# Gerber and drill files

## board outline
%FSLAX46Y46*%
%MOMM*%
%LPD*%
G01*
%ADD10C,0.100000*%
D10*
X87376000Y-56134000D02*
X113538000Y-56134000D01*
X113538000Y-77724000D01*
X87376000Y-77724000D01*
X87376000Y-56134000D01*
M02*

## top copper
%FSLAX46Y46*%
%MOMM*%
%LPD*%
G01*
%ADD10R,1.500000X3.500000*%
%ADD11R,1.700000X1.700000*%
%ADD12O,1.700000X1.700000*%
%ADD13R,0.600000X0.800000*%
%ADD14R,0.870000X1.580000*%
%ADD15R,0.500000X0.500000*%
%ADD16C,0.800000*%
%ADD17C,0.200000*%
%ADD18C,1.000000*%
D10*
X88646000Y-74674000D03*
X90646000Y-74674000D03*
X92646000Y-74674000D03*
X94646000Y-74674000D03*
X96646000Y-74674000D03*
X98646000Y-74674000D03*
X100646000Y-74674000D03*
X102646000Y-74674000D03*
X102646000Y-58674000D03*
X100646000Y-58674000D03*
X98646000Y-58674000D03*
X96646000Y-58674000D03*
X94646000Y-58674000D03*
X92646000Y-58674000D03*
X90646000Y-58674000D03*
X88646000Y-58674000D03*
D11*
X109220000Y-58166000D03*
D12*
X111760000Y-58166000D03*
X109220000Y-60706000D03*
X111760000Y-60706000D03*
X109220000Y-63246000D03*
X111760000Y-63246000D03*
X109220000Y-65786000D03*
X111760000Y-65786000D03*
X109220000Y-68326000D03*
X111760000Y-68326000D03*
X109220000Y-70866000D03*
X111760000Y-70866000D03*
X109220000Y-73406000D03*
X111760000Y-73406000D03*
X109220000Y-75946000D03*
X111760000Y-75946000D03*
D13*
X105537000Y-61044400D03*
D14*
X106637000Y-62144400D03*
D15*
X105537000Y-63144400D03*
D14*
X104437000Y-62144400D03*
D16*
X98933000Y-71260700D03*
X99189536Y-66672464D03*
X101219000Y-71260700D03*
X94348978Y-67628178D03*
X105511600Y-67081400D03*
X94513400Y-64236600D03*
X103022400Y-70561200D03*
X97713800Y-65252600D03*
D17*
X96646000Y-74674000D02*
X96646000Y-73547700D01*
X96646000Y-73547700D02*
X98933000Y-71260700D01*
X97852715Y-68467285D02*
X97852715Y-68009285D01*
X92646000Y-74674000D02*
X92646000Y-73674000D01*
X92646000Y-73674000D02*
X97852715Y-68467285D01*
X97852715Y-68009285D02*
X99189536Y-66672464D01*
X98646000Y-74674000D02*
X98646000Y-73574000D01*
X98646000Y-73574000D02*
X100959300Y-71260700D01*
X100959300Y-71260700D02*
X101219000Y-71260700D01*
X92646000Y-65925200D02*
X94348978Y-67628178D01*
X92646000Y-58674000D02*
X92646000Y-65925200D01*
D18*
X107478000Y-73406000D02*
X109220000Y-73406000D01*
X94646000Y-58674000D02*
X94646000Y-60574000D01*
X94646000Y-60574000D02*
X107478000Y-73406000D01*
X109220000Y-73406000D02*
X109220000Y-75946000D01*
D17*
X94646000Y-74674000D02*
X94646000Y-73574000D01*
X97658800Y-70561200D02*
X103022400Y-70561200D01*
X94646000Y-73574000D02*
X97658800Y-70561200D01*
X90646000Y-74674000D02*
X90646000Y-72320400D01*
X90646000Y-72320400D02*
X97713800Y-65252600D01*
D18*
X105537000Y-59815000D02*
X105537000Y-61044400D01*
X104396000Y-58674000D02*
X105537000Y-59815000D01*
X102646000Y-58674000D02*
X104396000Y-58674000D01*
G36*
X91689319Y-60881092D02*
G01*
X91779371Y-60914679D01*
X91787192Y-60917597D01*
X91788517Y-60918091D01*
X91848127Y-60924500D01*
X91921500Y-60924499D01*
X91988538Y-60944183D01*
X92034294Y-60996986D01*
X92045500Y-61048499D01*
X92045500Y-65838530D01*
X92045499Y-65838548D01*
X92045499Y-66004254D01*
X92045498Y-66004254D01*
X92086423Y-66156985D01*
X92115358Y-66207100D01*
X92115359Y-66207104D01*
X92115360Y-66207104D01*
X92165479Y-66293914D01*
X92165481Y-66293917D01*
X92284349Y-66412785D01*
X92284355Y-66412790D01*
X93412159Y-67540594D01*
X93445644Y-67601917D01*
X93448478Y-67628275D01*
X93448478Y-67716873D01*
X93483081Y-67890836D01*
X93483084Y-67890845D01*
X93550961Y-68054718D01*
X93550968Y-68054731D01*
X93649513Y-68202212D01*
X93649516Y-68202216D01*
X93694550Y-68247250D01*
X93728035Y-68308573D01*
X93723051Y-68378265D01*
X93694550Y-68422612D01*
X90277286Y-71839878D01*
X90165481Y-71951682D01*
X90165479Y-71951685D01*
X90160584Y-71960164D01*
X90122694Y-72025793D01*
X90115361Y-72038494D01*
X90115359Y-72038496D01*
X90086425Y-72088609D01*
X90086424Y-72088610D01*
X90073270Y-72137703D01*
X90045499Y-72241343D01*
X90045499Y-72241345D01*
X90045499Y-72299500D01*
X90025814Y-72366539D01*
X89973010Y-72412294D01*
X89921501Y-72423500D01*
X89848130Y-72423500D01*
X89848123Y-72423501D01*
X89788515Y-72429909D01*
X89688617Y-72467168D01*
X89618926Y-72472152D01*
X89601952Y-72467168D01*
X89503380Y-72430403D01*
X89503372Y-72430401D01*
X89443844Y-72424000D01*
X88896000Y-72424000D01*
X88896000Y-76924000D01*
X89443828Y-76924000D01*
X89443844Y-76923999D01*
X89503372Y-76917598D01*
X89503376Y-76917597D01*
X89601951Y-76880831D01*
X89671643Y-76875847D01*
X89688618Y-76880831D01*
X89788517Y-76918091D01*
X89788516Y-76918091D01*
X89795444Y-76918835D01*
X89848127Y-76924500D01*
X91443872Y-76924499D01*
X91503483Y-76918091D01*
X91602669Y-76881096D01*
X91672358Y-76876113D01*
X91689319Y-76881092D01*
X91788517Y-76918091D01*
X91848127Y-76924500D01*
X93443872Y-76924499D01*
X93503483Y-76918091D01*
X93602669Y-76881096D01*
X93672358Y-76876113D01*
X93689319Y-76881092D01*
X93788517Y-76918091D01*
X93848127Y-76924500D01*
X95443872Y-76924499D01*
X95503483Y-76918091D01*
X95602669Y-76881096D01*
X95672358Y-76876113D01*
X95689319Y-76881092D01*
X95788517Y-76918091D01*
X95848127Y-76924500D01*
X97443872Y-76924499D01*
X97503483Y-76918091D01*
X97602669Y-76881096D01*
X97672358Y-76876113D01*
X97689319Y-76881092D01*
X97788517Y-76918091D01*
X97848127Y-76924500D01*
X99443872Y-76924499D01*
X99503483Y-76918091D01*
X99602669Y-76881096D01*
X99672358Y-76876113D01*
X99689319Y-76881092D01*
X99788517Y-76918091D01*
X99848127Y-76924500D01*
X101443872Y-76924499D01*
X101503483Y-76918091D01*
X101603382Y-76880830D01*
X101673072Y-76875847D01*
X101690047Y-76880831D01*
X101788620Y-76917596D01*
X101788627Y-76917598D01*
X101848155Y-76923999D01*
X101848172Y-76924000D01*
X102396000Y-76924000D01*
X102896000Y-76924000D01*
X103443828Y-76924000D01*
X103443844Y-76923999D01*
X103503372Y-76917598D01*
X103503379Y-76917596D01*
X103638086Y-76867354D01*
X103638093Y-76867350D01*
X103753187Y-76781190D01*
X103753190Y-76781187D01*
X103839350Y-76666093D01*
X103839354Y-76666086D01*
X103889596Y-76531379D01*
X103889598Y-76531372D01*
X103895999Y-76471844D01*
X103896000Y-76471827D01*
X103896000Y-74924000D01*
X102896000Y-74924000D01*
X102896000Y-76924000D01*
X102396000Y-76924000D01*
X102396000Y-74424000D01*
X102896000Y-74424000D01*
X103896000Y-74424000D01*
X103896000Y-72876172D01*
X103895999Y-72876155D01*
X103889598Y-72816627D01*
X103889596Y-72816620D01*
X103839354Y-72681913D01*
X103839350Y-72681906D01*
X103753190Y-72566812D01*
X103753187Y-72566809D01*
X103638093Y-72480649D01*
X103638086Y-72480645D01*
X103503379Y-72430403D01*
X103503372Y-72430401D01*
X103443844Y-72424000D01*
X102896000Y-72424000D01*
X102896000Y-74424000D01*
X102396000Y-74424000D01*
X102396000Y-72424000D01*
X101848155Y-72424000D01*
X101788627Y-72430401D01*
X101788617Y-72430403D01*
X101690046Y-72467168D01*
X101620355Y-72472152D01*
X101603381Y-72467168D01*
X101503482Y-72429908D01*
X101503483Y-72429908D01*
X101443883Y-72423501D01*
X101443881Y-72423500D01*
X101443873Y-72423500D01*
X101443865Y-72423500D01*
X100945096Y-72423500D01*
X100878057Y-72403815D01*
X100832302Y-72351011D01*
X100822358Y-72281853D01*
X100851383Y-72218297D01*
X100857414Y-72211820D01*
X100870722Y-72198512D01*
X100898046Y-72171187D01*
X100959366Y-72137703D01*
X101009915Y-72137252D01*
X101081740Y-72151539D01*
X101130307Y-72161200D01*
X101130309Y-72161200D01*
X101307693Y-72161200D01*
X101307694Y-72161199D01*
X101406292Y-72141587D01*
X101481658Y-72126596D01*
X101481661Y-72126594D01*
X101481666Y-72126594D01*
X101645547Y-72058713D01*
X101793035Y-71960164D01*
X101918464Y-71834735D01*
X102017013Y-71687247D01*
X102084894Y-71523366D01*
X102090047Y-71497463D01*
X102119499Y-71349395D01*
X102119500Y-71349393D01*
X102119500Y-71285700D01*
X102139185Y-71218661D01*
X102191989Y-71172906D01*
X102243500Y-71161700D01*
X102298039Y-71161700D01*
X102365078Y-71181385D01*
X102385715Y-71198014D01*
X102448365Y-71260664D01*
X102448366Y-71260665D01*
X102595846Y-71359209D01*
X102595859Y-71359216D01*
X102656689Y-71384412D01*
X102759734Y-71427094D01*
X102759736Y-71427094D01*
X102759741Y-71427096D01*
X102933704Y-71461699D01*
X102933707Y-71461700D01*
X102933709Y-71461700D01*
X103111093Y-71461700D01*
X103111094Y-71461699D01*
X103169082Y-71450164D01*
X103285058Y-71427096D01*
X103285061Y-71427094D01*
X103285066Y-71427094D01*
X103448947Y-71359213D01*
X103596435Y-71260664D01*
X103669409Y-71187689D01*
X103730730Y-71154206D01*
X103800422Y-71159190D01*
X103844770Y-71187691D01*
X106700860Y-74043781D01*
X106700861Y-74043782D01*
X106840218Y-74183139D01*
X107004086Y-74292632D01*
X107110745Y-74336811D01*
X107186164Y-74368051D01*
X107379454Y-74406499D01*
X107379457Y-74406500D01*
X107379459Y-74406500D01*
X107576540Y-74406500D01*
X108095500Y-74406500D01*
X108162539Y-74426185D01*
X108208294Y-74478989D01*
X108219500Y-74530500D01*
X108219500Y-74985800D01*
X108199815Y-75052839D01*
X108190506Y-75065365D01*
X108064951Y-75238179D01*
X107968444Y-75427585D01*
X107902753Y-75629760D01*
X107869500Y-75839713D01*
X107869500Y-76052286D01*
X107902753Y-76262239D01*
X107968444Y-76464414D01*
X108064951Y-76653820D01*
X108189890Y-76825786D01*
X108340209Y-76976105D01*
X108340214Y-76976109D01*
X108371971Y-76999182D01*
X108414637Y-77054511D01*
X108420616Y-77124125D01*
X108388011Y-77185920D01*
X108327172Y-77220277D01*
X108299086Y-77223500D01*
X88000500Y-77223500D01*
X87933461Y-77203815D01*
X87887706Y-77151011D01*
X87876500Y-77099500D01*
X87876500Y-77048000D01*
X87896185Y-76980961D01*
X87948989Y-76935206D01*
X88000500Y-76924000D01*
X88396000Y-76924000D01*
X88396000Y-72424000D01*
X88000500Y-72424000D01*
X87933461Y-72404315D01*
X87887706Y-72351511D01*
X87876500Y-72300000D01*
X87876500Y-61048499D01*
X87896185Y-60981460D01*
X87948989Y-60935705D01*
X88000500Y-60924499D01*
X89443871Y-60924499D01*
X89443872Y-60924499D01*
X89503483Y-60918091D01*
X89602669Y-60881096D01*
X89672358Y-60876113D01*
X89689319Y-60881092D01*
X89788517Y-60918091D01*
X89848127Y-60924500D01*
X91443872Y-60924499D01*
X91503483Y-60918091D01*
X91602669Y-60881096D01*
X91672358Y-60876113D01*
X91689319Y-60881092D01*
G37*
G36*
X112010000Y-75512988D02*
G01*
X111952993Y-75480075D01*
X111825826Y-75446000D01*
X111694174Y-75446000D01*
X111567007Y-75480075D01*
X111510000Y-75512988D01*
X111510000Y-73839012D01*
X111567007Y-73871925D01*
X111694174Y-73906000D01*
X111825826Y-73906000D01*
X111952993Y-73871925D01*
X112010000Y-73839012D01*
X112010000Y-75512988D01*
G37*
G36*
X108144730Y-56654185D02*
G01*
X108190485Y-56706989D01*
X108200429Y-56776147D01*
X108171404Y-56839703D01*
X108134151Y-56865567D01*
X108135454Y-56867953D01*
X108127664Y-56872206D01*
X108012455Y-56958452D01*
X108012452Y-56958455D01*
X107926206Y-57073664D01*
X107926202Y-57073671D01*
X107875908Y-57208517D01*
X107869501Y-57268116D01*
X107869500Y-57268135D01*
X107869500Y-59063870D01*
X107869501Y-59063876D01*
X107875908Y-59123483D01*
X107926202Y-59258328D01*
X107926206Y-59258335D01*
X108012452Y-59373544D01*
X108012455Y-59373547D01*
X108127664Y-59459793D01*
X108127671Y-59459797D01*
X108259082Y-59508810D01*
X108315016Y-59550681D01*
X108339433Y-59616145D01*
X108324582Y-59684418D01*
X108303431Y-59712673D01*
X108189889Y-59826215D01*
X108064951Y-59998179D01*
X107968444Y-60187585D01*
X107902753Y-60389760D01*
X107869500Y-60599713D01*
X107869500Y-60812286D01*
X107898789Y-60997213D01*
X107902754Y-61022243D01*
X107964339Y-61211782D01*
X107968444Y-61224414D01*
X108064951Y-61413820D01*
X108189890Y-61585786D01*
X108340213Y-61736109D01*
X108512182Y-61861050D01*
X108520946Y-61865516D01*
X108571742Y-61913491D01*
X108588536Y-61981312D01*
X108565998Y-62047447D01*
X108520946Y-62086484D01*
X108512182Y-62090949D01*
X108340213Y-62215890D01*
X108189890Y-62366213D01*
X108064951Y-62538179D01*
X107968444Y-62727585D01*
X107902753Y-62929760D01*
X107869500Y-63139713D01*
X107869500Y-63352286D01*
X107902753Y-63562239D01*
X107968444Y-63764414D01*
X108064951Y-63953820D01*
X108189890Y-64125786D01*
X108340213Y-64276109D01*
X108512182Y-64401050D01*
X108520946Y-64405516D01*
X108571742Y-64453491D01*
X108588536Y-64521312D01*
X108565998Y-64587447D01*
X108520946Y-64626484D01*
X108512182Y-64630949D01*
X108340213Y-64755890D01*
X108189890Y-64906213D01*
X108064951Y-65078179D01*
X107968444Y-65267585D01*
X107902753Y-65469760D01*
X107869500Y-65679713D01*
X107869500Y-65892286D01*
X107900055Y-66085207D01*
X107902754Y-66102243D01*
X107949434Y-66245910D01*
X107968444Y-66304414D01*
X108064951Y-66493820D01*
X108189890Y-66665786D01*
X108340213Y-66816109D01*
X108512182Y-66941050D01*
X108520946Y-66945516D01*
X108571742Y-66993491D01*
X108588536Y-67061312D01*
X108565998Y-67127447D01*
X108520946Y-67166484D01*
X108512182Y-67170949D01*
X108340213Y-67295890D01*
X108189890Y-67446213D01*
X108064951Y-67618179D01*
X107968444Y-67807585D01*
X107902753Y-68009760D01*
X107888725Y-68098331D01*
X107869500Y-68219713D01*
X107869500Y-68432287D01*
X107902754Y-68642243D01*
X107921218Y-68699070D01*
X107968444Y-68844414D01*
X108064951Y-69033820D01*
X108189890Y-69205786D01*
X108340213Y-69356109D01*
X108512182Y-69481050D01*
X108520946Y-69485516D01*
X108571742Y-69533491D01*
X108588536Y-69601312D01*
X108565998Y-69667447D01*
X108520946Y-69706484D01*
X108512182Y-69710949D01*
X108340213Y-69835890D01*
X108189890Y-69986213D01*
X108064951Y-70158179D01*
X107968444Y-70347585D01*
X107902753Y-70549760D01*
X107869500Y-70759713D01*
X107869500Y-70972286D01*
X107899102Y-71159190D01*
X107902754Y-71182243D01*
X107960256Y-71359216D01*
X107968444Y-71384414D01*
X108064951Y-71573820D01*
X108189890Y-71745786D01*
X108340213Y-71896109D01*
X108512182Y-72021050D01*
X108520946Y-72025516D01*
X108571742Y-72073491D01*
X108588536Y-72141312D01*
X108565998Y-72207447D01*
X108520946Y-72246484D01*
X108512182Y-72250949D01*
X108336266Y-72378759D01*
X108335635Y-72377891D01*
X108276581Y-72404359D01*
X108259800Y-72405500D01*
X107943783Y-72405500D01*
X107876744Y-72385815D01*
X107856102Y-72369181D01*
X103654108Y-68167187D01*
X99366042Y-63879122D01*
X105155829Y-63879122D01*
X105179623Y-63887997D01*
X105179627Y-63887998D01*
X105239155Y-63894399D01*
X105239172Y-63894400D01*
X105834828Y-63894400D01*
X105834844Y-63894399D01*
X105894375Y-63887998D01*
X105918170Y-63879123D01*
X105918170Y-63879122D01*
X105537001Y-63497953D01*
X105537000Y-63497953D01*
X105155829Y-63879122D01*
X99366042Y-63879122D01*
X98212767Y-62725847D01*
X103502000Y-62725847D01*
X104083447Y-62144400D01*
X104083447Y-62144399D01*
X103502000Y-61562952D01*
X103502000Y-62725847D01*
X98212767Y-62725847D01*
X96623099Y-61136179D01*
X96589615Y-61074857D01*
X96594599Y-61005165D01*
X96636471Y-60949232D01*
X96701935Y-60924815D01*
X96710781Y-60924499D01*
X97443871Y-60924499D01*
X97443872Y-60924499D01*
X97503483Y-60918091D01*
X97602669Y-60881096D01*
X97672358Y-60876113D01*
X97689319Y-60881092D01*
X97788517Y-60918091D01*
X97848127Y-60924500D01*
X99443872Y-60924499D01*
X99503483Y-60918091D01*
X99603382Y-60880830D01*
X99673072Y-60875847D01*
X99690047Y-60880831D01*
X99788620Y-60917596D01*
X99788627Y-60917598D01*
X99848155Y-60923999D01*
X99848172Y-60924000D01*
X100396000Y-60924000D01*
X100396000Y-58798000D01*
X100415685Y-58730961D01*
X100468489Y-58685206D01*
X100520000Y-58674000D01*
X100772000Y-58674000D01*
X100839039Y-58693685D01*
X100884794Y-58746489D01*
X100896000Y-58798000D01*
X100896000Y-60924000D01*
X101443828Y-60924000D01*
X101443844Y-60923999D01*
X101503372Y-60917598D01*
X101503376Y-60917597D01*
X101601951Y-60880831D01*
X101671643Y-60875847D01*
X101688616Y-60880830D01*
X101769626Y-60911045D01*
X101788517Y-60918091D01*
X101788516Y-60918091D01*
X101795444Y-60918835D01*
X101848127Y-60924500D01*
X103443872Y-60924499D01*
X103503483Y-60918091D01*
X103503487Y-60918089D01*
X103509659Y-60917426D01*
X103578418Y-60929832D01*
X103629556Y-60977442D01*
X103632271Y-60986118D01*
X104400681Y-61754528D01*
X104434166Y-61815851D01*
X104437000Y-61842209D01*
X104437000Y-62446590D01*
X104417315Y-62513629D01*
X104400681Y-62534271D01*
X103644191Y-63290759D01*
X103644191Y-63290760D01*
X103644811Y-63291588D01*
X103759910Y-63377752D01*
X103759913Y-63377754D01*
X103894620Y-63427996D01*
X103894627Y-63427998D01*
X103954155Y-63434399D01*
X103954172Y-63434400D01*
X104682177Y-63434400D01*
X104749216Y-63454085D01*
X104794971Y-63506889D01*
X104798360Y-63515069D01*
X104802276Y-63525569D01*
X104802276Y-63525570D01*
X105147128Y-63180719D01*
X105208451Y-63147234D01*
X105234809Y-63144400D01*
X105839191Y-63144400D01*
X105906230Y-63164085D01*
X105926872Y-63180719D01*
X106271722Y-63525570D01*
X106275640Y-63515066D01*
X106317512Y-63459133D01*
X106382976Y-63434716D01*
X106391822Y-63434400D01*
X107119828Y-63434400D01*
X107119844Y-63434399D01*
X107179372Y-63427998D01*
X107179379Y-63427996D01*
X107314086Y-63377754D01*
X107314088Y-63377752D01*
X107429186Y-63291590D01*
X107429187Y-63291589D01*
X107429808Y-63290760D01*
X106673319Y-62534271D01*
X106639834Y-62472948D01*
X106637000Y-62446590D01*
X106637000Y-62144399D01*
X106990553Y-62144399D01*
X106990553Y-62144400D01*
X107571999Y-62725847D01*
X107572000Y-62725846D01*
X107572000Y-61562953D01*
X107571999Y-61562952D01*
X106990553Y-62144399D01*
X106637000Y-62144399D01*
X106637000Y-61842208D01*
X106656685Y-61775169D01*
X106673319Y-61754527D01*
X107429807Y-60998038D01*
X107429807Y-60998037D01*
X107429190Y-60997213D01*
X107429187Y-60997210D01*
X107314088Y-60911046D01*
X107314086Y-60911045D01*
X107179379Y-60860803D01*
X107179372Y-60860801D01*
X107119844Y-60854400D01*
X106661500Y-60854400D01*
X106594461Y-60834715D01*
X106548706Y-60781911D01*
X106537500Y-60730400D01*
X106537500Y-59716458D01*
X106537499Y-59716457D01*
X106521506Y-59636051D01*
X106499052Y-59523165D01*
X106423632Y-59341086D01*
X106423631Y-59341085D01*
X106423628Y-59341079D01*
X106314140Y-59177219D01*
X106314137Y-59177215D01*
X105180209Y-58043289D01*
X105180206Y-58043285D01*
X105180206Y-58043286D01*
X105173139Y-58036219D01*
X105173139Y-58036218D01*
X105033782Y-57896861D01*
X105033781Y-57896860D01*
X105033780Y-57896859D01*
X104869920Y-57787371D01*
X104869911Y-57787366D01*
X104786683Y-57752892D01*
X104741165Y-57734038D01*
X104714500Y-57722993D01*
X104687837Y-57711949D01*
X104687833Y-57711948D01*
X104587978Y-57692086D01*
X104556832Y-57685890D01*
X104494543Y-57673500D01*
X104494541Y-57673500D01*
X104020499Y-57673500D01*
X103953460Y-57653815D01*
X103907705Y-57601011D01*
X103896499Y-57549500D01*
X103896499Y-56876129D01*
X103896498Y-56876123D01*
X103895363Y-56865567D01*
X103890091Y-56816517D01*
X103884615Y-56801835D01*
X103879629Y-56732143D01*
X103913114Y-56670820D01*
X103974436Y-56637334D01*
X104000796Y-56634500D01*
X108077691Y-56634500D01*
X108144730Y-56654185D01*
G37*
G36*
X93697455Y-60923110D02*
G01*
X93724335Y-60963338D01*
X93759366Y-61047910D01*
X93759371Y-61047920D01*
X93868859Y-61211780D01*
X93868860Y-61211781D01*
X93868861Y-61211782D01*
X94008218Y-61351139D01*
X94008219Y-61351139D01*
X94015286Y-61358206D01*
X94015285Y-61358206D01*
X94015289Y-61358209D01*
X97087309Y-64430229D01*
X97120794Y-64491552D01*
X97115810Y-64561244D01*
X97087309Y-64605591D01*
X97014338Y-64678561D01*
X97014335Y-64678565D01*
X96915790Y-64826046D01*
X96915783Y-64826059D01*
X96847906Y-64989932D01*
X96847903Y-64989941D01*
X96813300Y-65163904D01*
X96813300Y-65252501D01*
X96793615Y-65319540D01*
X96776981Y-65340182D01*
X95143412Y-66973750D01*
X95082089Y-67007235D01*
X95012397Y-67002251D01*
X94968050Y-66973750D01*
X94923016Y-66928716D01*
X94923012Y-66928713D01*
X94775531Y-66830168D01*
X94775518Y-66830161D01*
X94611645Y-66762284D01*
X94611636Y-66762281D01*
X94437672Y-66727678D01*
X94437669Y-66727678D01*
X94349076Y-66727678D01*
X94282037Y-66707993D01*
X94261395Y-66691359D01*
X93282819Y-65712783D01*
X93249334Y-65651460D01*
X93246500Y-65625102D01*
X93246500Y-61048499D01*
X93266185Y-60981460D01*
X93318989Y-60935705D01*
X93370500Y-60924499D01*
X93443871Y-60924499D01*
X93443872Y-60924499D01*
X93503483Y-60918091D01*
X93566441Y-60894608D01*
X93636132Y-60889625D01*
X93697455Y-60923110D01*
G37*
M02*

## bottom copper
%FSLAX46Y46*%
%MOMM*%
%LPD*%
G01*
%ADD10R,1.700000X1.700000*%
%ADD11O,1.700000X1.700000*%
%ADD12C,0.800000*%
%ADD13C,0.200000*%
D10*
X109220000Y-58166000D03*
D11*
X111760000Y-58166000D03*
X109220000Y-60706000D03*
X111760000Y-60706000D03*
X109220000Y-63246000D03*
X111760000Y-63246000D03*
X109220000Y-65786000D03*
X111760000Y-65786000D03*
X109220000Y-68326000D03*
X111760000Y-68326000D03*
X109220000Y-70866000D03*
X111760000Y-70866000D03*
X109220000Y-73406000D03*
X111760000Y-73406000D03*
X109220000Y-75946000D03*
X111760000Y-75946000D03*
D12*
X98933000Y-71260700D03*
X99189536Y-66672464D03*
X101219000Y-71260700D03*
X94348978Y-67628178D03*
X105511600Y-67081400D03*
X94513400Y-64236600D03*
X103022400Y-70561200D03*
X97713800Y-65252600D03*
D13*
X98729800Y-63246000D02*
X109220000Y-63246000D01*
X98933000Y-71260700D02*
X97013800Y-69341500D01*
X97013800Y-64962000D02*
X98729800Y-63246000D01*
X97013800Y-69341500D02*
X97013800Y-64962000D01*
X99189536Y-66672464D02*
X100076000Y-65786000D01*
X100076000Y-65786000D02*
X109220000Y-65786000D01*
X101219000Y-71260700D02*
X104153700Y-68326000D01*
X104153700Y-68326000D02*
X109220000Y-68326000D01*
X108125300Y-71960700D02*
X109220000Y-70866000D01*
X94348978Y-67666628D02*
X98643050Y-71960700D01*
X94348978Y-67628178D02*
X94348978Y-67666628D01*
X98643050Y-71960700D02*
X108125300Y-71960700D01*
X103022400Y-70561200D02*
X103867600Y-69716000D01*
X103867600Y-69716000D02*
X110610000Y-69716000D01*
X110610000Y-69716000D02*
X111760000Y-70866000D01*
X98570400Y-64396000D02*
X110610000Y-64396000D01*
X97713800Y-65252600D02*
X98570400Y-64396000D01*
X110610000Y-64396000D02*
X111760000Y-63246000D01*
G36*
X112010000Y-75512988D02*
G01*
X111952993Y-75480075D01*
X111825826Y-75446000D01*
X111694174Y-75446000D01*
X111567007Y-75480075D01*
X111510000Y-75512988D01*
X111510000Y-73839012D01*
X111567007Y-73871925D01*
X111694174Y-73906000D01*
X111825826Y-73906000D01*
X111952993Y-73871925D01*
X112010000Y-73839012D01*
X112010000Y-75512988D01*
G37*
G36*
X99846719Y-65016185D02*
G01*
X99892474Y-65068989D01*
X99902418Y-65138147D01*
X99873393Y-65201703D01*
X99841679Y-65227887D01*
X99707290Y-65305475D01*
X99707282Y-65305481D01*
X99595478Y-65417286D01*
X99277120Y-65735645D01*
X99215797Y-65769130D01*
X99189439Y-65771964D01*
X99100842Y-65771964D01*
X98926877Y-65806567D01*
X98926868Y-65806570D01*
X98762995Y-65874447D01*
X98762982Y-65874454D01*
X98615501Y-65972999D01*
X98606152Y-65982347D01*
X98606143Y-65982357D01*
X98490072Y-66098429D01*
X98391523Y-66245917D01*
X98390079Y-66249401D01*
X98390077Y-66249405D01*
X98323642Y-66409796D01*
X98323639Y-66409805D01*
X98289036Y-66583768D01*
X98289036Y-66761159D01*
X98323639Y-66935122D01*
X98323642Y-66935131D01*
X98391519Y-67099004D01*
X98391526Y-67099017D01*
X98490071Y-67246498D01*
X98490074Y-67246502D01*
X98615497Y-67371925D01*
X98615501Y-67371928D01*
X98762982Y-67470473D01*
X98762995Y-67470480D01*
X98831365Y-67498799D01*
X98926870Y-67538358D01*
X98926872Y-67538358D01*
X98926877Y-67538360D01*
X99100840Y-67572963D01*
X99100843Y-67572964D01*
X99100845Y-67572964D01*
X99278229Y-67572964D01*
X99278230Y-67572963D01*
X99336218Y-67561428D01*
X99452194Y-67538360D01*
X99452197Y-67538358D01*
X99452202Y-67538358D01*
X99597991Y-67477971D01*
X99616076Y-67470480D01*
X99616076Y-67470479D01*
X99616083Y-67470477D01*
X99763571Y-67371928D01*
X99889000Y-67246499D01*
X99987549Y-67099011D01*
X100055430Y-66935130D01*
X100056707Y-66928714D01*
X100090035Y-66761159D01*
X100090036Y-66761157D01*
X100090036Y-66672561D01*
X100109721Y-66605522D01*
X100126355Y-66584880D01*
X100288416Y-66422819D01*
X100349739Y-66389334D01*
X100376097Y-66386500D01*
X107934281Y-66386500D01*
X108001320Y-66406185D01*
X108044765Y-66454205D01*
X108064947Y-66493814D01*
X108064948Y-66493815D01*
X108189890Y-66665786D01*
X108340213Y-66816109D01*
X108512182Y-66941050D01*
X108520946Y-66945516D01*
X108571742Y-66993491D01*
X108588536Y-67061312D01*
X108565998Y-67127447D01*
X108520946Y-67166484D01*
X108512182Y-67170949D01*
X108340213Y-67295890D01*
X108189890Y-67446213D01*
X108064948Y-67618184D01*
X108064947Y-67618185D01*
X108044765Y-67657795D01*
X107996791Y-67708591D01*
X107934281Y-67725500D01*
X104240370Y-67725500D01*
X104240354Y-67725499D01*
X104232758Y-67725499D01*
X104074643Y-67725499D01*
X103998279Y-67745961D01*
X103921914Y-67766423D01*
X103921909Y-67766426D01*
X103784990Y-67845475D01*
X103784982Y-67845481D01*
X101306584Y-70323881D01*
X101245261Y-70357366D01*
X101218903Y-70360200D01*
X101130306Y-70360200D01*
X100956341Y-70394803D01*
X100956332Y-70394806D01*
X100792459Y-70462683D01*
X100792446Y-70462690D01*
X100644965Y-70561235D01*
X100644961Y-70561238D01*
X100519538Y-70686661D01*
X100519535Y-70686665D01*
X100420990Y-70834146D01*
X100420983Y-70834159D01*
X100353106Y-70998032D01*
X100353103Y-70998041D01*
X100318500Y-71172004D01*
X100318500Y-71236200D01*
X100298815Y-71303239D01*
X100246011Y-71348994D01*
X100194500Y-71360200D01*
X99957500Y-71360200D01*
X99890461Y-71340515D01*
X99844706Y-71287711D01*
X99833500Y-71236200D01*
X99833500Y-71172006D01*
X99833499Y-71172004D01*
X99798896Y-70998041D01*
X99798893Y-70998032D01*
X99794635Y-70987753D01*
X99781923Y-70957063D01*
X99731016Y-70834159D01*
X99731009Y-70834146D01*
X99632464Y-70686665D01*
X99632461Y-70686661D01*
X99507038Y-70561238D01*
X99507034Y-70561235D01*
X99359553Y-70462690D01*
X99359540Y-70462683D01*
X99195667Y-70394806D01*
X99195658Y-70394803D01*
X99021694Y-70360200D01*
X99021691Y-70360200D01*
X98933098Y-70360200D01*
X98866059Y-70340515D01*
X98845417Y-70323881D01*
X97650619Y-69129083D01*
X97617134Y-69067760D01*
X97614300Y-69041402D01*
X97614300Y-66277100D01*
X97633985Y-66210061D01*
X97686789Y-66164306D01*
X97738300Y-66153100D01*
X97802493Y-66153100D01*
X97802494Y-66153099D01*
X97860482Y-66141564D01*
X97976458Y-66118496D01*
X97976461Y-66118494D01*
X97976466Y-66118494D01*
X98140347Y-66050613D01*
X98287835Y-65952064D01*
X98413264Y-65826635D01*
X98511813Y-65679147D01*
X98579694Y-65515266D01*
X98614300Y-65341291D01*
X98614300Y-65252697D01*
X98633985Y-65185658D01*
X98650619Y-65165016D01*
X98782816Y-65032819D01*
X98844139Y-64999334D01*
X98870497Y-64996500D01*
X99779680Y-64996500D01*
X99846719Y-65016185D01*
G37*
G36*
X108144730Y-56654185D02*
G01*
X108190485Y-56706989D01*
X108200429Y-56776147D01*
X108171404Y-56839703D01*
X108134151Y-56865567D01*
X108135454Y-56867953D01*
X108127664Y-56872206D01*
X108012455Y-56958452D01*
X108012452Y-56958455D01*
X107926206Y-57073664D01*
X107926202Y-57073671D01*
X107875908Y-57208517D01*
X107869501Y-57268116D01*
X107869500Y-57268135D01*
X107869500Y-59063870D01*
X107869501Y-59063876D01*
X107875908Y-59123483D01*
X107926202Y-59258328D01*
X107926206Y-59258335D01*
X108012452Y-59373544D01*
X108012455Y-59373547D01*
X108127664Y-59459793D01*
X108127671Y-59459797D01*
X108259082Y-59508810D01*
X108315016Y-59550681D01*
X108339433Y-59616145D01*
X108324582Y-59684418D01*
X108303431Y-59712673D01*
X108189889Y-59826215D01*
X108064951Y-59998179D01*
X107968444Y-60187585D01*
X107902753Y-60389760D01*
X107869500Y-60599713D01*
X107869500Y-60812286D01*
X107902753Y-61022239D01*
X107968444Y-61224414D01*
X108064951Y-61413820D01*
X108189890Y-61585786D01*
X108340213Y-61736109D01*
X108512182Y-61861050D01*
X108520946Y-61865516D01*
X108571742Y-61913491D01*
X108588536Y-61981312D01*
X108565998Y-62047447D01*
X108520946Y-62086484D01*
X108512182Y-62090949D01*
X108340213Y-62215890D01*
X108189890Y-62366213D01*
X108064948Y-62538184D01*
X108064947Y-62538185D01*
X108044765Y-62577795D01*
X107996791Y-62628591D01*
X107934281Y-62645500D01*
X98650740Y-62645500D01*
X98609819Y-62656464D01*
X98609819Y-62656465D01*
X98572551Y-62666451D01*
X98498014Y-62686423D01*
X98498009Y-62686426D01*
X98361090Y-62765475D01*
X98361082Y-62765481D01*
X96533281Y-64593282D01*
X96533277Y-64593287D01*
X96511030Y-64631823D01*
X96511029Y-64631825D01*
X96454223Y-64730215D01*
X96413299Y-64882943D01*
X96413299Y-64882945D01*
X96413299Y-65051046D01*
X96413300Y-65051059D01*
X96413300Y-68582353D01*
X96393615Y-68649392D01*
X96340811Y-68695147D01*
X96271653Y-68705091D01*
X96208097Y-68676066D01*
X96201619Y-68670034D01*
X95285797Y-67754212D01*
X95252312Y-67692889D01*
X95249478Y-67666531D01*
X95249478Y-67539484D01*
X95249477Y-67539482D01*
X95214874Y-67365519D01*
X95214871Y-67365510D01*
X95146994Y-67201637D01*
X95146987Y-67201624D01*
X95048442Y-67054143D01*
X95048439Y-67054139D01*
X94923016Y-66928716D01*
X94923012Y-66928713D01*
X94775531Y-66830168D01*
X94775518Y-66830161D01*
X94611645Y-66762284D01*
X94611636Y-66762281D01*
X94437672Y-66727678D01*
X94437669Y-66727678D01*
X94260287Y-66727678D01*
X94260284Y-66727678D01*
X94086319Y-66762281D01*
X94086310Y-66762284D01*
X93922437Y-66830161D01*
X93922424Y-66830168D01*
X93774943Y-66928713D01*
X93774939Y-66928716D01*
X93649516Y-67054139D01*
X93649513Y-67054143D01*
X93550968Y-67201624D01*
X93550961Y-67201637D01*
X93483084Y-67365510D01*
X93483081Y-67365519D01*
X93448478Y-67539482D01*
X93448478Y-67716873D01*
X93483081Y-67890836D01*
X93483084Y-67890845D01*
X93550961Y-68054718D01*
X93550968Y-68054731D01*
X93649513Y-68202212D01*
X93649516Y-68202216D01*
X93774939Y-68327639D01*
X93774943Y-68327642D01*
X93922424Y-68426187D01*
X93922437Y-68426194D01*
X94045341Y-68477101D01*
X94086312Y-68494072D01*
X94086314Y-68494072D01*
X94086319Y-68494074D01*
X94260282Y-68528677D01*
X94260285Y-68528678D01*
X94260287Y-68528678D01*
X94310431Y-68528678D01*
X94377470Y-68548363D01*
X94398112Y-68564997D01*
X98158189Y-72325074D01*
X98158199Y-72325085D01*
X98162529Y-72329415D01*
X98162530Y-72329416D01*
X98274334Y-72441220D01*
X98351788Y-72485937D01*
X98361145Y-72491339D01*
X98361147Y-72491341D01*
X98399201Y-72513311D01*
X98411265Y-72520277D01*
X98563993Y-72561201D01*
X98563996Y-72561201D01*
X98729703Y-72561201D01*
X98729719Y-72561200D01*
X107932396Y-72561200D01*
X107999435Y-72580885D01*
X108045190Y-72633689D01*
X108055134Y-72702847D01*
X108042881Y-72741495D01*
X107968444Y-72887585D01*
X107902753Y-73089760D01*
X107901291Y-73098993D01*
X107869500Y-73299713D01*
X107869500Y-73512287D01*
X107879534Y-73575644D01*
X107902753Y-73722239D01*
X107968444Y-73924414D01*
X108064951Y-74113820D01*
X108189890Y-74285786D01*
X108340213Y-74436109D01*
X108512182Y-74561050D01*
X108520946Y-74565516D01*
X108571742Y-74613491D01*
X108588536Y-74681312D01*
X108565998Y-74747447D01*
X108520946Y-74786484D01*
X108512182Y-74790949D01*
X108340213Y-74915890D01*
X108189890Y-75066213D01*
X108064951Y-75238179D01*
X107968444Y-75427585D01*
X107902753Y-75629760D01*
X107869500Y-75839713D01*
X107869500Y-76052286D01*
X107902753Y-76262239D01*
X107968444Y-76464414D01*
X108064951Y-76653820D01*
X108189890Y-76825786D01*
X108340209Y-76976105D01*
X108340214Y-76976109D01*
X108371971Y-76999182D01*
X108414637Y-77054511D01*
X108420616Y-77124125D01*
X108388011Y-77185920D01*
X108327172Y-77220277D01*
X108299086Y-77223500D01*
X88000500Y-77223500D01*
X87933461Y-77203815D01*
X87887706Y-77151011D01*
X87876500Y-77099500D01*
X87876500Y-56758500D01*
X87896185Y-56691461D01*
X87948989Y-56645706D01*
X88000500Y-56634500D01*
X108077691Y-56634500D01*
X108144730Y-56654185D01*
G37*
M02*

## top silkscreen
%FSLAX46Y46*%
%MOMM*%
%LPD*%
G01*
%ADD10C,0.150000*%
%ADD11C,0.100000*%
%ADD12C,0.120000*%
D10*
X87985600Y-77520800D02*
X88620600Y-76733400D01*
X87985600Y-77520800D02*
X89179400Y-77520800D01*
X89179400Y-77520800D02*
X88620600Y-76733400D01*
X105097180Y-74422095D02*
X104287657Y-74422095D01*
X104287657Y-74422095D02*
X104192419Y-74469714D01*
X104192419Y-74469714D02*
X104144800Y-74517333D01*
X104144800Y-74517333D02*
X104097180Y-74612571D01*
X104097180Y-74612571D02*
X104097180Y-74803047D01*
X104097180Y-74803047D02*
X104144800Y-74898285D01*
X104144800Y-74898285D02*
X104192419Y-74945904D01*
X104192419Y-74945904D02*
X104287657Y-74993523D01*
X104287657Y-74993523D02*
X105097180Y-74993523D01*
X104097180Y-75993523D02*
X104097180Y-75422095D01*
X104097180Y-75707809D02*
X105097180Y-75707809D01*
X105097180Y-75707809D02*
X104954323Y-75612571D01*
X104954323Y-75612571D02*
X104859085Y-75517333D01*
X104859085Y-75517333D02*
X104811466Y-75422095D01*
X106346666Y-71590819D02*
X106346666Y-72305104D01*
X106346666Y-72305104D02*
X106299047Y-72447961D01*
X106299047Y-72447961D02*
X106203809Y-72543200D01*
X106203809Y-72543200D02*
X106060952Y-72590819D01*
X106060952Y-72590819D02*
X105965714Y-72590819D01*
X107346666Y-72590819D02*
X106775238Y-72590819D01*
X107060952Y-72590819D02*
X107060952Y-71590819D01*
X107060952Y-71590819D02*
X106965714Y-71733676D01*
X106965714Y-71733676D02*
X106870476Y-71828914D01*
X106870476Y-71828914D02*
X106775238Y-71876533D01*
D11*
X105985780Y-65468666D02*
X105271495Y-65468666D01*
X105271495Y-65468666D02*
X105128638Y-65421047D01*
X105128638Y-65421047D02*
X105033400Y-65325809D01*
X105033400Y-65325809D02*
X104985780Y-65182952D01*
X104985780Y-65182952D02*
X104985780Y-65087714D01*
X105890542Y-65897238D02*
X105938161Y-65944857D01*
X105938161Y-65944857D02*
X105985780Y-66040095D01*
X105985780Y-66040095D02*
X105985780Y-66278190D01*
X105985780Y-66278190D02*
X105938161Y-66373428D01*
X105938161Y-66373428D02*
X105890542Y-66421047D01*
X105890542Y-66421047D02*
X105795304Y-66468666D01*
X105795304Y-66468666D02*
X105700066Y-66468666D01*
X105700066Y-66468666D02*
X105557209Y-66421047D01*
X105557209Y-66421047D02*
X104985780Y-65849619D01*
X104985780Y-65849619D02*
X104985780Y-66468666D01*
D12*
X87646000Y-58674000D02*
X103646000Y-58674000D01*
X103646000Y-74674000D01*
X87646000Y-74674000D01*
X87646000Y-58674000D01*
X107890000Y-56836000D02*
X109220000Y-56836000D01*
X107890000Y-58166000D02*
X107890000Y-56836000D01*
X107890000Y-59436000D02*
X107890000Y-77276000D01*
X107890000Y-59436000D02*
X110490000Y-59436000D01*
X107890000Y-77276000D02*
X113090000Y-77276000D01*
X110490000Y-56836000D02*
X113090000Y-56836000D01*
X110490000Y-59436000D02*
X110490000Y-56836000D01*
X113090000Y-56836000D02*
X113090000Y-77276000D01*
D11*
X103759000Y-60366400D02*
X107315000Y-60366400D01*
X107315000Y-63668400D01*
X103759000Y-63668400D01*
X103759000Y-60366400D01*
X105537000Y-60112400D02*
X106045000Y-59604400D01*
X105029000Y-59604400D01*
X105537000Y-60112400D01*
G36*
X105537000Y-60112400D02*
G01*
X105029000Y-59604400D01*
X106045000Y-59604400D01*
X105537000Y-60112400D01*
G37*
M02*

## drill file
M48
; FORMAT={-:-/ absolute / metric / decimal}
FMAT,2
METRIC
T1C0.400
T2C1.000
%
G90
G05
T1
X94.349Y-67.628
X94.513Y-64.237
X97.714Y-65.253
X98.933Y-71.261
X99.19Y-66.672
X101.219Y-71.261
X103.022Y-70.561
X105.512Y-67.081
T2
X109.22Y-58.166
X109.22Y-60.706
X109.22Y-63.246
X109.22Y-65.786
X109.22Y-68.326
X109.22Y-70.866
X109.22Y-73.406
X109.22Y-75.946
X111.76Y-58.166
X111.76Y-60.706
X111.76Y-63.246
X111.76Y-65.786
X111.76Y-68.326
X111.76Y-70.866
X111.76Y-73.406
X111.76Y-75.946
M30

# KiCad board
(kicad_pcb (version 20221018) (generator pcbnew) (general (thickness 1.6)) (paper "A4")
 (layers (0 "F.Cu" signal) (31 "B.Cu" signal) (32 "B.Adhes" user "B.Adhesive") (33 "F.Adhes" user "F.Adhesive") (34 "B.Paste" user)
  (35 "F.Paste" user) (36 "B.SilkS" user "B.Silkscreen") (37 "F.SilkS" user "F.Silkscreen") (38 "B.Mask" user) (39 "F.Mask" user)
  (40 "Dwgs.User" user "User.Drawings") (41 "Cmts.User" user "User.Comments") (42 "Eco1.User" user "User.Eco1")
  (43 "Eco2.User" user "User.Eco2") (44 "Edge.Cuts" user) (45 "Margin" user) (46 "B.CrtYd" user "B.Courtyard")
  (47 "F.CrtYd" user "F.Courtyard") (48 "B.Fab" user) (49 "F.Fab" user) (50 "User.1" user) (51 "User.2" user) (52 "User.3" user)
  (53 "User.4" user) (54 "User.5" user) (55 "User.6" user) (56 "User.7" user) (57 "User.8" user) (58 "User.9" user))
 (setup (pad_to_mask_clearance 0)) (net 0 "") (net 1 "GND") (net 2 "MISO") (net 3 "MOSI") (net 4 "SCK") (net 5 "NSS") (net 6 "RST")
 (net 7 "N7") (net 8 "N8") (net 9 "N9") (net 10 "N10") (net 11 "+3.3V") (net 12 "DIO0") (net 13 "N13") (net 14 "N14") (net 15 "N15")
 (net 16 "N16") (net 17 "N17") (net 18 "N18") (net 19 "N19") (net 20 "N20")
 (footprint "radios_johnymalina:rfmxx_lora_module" (layer "F.Cu") (at 95.646 66.674 90)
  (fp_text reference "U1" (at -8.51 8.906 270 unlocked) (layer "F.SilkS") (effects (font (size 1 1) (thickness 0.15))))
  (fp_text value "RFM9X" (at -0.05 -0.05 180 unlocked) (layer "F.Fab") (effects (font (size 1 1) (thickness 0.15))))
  (fp_rect (start -8 8) (end 8 -8) (stroke (width 0.12) (type solid)) (fill none) (layer "F.SilkS"))
  (pad "1" smd rect (at -8 -7 90) (size 3.5 1.5) (layers "F.Cu" "F.Paste" "F.Mask") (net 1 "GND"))
  (pad "2" smd rect (at -8 -5 90) (size 3.5 1.5) (layers "F.Cu" "F.Paste" "F.Mask") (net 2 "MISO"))
  (pad "3" smd rect (at -8 -3 90) (size 3.5 1.5) (layers "F.Cu" "F.Paste" "F.Mask") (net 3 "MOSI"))
  (pad "4" smd rect (at -8 -1 90) (size 3.5 1.5) (layers "F.Cu" "F.Paste" "F.Mask") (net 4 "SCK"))
  (pad "5" smd rect (at -8 1 90) (size 3.5 1.5) (layers "F.Cu" "F.Paste" "F.Mask") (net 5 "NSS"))
  (pad "6" smd rect (at -8 3 90) (size 3.5 1.5) (layers "F.Cu" "F.Paste" "F.Mask") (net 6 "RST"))
  (pad "7" smd rect (at -8 5 90) (size 3.5 1.5) (layers "F.Cu" "F.Paste" "F.Mask") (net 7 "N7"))
  (pad "8" smd rect (at -8 7 90) (size 3.5 1.5) (layers "F.Cu" "F.Paste" "F.Mask") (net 1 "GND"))
  (pad "9" smd rect (at 8 7 90) (size 3.5 1.5) (layers "F.Cu" "F.Paste" "F.Mask") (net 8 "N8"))
  (pad "10" smd rect (at 8 5 90) (size 3.5 1.5) (layers "F.Cu" "F.Paste" "F.Mask") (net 1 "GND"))
  (pad "11" smd rect (at 8 3 90) (size 3.5 1.5) (layers "F.Cu" "F.Paste" "F.Mask") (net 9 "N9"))
  (pad "12" smd rect (at 8 1 90) (size 3.5 1.5) (layers "F.Cu" "F.Paste" "F.Mask") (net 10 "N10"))
  (pad "13" smd rect (at 8 -1 90) (size 3.5 1.5) (layers "F.Cu" "F.Paste" "F.Mask") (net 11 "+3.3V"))
  (pad "14" smd rect (at 8 -3 90) (size 3.5 1.5) (layers "F.Cu" "F.Paste" "F.Mask") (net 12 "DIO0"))
  (pad "15" smd rect (at 8 -5 90) (size 3.5 1.5) (layers "F.Cu" "F.Paste" "F.Mask") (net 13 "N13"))
  (pad "16" smd rect (at 8 -7 90) (size 3.5 1.5) (layers "F.Cu" "F.Paste" "F.Mask") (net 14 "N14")))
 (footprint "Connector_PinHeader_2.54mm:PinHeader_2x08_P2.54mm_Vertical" (layer "F.Cu") (at 109.22 58.166)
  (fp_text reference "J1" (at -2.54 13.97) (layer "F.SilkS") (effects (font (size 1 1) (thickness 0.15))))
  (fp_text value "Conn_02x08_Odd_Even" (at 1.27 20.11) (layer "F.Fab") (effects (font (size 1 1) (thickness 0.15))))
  (fp_line (start -1.33 -1.33) (end 0 -1.33) (stroke (width 0.12) (type solid)) (layer "F.SilkS"))
  (fp_line (start -1.33 0) (end -1.33 -1.33) (stroke (width 0.12) (type solid)) (layer "F.SilkS"))
  (fp_line (start -1.33 1.27) (end -1.33 19.11) (stroke (width 0.12) (type solid)) (layer "F.SilkS"))
  (fp_line (start -1.33 1.27) (end 1.27 1.27) (stroke (width 0.12) (type solid)) (layer "F.SilkS"))
  (fp_line (start -1.33 19.11) (end 3.87 19.11) (stroke (width 0.12) (type solid)) (layer "F.SilkS"))
  (fp_line (start 1.27 -1.33) (end 3.87 -1.33) (stroke (width 0.12) (type solid)) (layer "F.SilkS"))
  (fp_line (start 1.27 1.27) (end 1.27 -1.33) (stroke (width 0.12) (type solid)) (layer "F.SilkS"))
  (fp_line (start 3.87 -1.33) (end 3.87 19.11) (stroke (width 0.12) (type solid)) (layer "F.SilkS"))
  (pad "1" thru_hole rect (at 0 0) (size 1.7 1.7) (drill 1) (layers "*.Cu" "*.Mask") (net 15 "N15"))
  (pad "2" thru_hole oval (at 2.54 0) (size 1.7 1.7) (drill 1) (layers "*.Cu" "*.Mask") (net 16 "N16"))
  (pad "3" thru_hole oval (at 0 2.54) (size 1.7 1.7) (drill 1) (layers "*.Cu" "*.Mask") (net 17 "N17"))
  (pad "4" thru_hole oval (at 2.54 2.54) (size 1.7 1.7) (drill 1) (layers "*.Cu" "*.Mask") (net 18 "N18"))
  (pad "5" thru_hole oval (at 0 5.08) (size 1.7 1.7) (drill 1) (layers "*.Cu" "*.Mask") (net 5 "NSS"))
  (pad "6" thru_hole oval (at 2.54 5.08) (size 1.7 1.7) (drill 1) (layers "*.Cu" "*.Mask") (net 2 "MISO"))
  (pad "7" thru_hole oval (at 0 7.62) (size 1.7 1.7) (drill 1) (layers "*.Cu" "*.Mask") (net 3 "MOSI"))
  (pad "8" thru_hole oval (at 2.54 7.62) (size 1.7 1.7) (drill 1) (layers "*.Cu" "*.Mask") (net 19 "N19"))
  (pad "9" thru_hole oval (at 0 10.16) (size 1.7 1.7) (drill 1) (layers "*.Cu" "*.Mask") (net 6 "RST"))
  (pad "10" thru_hole oval (at 2.54 10.16) (size 1.7 1.7) (drill 1) (layers "*.Cu" "*.Mask") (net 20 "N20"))
  (pad "11" thru_hole oval (at 0 12.7) (size 1.7 1.7) (drill 1) (layers "*.Cu" "*.Mask") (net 12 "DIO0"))
  (pad "12" thru_hole oval (at 2.54 12.7) (size 1.7 1.7) (drill 1) (layers "*.Cu" "*.Mask") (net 4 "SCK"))
  (pad "13" thru_hole oval (at 0 15.24) (size 1.7 1.7) (drill 1) (layers "*.Cu" "*.Mask") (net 11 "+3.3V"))
  (pad "14" thru_hole oval (at 2.54 15.24) (size 1.7 1.7) (drill 1) (layers "*.Cu" "*.Mask") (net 1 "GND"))
  (pad "15" thru_hole oval (at 0 17.78) (size 1.7 1.7) (drill 1) (layers "*.Cu" "*.Mask") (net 11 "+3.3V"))
  (pad "16" thru_hole oval (at 2.54 17.78) (size 1.7 1.7) (drill 1) (layers "*.Cu" "*.Mask") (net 1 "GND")))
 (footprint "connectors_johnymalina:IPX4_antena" (layer "F.Cu") (at 105.537 62.1444 180)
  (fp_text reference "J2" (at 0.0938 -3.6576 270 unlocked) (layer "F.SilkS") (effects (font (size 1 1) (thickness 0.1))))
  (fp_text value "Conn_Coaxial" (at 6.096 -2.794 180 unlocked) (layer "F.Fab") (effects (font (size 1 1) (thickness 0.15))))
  (fp_rect (start -1.778 -1.524) (end 1.778 1.778) (stroke (width 0.1) (type default)) (fill none) (layer "F.SilkS"))
  (fp_poly (pts (xy 0 2.032) (xy -0.508 2.54) (xy 0.508 2.54)) (stroke (width 0.1) (type solid)) (fill solid) (layer "F.SilkS"))
  (pad "1" smd rect (at 0 1.1 180) (size 0.6 0.8) (layers "F.Cu" "F.Paste" "F.Mask") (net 8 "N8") (thermal_bridge_angle 45))
  (pad "2" smd rect (at -1.1 0 180) (size 0.87 1.58) (layers "F.Cu" "F.Paste" "F.Mask") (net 1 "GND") (thermal_bridge_angle 45))
  (pad "2" smd rect (at 0 -1 180) (size 0.5 0.5) (layers "F.Cu" "F.Paste" "F.Mask") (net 1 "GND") (thermal_bridge_angle 45))
  (pad "2" smd rect (at 1.1 0 180) (size 0.87 1.58) (layers "F.Cu" "F.Paste" "F.Mask") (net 1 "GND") (thermal_bridge_angle 45)))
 (gr_line (start 87.9856 77.5208) (end 88.6206 76.7334) (stroke (width 0.15) (type default)) (layer "F.SilkS"))
 (gr_line (start 87.9856 77.5208) (end 89.1794 77.5208) (stroke (width 0.15) (type default)) (layer "F.SilkS"))
 (gr_line (start 89.1794 77.5208) (end 88.6206 76.7334) (stroke (width 0.15) (type default)) (layer "F.SilkS"))
 (gr_rect (start 87.376 56.134) (end 113.538 77.724) (stroke (width 0.1) (type default)) (fill none) (layer "Edge.Cuts"))
 (segment (start 96.646 74.674) (end 96.646 73.5477) (width 0.2) (layer "F.Cu") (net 5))
 (segment (start 96.646 73.5477) (end 98.933 71.2607) (width 0.2) (layer "F.Cu") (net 5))
 (via (at 98.933 71.2607) (size 0.8) (drill 0.4) (layers "F.Cu" "B.Cu") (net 5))
 (segment (start 98.7298 63.246) (end 109.22 63.246) (width 0.2) (layer "B.Cu") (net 5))
 (segment (start 98.933 71.2607) (end 97.0138 69.3415) (width 0.2) (layer "B.Cu") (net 5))
 (segment (start 97.0138 64.962) (end 98.7298 63.246) (width 0.2) (layer "B.Cu") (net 5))
 (segment (start 97.0138 69.3415) (end 97.0138 64.962) (width 0.2) (layer "B.Cu") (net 5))
 (segment (start 97.852715 68.467285) (end 97.852715 68.009285) (width 0.2) (layer "F.Cu") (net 3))
 (segment (start 92.646 74.674) (end 92.646 73.674) (width 0.2) (layer "F.Cu") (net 3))
 (segment (start 92.646 73.674) (end 97.852715 68.467285) (width 0.2) (layer "F.Cu") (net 3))
 (segment (start 97.852715 68.009285) (end 99.189536 66.672464) (width 0.2) (layer "F.Cu") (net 3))
 (via (at 99.189536 66.672464) (size 0.8) (drill 0.4) (layers "F.Cu" "B.Cu") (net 3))
 (segment (start 99.189536 66.672464) (end 100.076 65.786) (width 0.2) (layer "B.Cu") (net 3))
 (segment (start 100.076 65.786) (end 109.22 65.786) (width 0.2) (layer "B.Cu") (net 3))
 (segment (start 98.646 74.674) (end 98.646 73.574) (width 0.2) (layer "F.Cu") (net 6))
 (segment (start 98.646 73.574) (end 100.9593 71.2607) (width 0.2) (layer "F.Cu") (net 6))
 (segment (start 100.9593 71.2607) (end 101.219 71.2607) (width 0.2) (layer "F.Cu") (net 6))
 (via (at 101.219 71.2607) (size 0.8) (drill 0.4) (layers "F.Cu" "B.Cu") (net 6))
 (segment (start 101.219 71.2607) (end 104.1537 68.326) (width 0.2) (layer "B.Cu") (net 6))
 (segment (start 104.1537 68.326) (end 109.22 68.326) (width 0.2) (layer "B.Cu") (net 6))
 (segment (start 92.646 65.9252) (end 94.348978 67.628178) (width 0.2) (layer "F.Cu") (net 12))
 (segment (start 92.646 58.674) (end 92.646 65.9252) (width 0.2) (layer "F.Cu") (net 12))
 (via (at 94.348978 67.628178) (size 0.8) (drill 0.4) (layers "F.Cu" "B.Cu") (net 12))
 (segment (start 108.1253 71.9607) (end 109.22 70.866) (width 0.2) (layer "B.Cu") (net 12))
 (segment (start 94.348978 67.666628) (end 98.64305 71.9607) (width 0.2) (layer "B.Cu") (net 12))
 (segment (start 94.348978 67.628178) (end 94.348978 67.666628) (width 0.2) (layer "B.Cu") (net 12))
 (segment (start 98.64305 71.9607) (end 108.1253 71.9607) (width 0.2) (layer "B.Cu") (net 12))
 (segment (start 107.478 73.406) (end 109.22 73.406) (width 1) (layer "F.Cu") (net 11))
 (segment (start 94.646 58.674) (end 94.646 60.574) (width 1) (layer "F.Cu") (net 11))
 (segment (start 94.646 60.574) (end 107.478 73.406) (width 1) (layer "F.Cu") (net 11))
 (segment (start 109.22 73.406) (end 109.22 75.946) (width 1) (layer "F.Cu") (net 11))
 (via (at 105.5116 67.0814) (size 0.8) (drill 0.4) (layers "F.Cu" "B.Cu") (free) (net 1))
 (via (at 94.5134 64.2366) (size 0.8) (drill 0.4) (layers "F.Cu" "B.Cu") (free) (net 1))
 (segment (start 94.646 74.674) (end 94.646 73.574) (width 0.2) (layer "F.Cu") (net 4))
 (segment (start 97.6588 70.5612) (end 103.0224 70.5612) (width 0.2) (layer "F.Cu") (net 4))
 (segment (start 94.646 73.574) (end 97.6588 70.5612) (width 0.2) (layer "F.Cu") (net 4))
 (via (at 103.0224 70.5612) (size 0.8) (drill 0.4) (layers "F.Cu" "B.Cu") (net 4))
 (segment (start 103.0224 70.5612) (end 103.8676 69.716) (width 0.2) (layer "B.Cu") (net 4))
 (segment (start 103.8676 69.716) (end 110.61 69.716) (width 0.2) (layer "B.Cu") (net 4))
 (segment (start 110.61 69.716) (end 111.76 70.866) (width 0.2) (layer "B.Cu") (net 4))
 (segment (start 90.646 74.674) (end 90.646 72.3204) (width 0.2) (layer "F.Cu") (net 2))
 (segment (start 90.646 72.3204) (end 97.7138 65.2526) (width 0.2) (layer "F.Cu") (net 2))
 (via (at 97.7138 65.2526) (size 0.8) (drill 0.4) (layers "F.Cu" "B.Cu") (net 2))
 (segment (start 98.5704 64.396) (end 110.61 64.396) (width 0.2) (layer "B.Cu") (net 2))
 (segment (start 97.7138 65.2526) (end 98.5704 64.396) (width 0.2) (layer "B.Cu") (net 2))
 (segment (start 110.61 64.396) (end 111.76 63.246) (width 0.2) (layer "B.Cu") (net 2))
 (segment (start 105.537 59.815) (end 105.537 61.0444) (width 1) (layer "F.Cu") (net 8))
 (segment (start 104.396 58.674) (end 105.537 59.815) (width 1) (layer "F.Cu") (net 8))
 (segment (start 102.646 58.674) (end 104.396 58.674) (width 1) (layer "F.Cu") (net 8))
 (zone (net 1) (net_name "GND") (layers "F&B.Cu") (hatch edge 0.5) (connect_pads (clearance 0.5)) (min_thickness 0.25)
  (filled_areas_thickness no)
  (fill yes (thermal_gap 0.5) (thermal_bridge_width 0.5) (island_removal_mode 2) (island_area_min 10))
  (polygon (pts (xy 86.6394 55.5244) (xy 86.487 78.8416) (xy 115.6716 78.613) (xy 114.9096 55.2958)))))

